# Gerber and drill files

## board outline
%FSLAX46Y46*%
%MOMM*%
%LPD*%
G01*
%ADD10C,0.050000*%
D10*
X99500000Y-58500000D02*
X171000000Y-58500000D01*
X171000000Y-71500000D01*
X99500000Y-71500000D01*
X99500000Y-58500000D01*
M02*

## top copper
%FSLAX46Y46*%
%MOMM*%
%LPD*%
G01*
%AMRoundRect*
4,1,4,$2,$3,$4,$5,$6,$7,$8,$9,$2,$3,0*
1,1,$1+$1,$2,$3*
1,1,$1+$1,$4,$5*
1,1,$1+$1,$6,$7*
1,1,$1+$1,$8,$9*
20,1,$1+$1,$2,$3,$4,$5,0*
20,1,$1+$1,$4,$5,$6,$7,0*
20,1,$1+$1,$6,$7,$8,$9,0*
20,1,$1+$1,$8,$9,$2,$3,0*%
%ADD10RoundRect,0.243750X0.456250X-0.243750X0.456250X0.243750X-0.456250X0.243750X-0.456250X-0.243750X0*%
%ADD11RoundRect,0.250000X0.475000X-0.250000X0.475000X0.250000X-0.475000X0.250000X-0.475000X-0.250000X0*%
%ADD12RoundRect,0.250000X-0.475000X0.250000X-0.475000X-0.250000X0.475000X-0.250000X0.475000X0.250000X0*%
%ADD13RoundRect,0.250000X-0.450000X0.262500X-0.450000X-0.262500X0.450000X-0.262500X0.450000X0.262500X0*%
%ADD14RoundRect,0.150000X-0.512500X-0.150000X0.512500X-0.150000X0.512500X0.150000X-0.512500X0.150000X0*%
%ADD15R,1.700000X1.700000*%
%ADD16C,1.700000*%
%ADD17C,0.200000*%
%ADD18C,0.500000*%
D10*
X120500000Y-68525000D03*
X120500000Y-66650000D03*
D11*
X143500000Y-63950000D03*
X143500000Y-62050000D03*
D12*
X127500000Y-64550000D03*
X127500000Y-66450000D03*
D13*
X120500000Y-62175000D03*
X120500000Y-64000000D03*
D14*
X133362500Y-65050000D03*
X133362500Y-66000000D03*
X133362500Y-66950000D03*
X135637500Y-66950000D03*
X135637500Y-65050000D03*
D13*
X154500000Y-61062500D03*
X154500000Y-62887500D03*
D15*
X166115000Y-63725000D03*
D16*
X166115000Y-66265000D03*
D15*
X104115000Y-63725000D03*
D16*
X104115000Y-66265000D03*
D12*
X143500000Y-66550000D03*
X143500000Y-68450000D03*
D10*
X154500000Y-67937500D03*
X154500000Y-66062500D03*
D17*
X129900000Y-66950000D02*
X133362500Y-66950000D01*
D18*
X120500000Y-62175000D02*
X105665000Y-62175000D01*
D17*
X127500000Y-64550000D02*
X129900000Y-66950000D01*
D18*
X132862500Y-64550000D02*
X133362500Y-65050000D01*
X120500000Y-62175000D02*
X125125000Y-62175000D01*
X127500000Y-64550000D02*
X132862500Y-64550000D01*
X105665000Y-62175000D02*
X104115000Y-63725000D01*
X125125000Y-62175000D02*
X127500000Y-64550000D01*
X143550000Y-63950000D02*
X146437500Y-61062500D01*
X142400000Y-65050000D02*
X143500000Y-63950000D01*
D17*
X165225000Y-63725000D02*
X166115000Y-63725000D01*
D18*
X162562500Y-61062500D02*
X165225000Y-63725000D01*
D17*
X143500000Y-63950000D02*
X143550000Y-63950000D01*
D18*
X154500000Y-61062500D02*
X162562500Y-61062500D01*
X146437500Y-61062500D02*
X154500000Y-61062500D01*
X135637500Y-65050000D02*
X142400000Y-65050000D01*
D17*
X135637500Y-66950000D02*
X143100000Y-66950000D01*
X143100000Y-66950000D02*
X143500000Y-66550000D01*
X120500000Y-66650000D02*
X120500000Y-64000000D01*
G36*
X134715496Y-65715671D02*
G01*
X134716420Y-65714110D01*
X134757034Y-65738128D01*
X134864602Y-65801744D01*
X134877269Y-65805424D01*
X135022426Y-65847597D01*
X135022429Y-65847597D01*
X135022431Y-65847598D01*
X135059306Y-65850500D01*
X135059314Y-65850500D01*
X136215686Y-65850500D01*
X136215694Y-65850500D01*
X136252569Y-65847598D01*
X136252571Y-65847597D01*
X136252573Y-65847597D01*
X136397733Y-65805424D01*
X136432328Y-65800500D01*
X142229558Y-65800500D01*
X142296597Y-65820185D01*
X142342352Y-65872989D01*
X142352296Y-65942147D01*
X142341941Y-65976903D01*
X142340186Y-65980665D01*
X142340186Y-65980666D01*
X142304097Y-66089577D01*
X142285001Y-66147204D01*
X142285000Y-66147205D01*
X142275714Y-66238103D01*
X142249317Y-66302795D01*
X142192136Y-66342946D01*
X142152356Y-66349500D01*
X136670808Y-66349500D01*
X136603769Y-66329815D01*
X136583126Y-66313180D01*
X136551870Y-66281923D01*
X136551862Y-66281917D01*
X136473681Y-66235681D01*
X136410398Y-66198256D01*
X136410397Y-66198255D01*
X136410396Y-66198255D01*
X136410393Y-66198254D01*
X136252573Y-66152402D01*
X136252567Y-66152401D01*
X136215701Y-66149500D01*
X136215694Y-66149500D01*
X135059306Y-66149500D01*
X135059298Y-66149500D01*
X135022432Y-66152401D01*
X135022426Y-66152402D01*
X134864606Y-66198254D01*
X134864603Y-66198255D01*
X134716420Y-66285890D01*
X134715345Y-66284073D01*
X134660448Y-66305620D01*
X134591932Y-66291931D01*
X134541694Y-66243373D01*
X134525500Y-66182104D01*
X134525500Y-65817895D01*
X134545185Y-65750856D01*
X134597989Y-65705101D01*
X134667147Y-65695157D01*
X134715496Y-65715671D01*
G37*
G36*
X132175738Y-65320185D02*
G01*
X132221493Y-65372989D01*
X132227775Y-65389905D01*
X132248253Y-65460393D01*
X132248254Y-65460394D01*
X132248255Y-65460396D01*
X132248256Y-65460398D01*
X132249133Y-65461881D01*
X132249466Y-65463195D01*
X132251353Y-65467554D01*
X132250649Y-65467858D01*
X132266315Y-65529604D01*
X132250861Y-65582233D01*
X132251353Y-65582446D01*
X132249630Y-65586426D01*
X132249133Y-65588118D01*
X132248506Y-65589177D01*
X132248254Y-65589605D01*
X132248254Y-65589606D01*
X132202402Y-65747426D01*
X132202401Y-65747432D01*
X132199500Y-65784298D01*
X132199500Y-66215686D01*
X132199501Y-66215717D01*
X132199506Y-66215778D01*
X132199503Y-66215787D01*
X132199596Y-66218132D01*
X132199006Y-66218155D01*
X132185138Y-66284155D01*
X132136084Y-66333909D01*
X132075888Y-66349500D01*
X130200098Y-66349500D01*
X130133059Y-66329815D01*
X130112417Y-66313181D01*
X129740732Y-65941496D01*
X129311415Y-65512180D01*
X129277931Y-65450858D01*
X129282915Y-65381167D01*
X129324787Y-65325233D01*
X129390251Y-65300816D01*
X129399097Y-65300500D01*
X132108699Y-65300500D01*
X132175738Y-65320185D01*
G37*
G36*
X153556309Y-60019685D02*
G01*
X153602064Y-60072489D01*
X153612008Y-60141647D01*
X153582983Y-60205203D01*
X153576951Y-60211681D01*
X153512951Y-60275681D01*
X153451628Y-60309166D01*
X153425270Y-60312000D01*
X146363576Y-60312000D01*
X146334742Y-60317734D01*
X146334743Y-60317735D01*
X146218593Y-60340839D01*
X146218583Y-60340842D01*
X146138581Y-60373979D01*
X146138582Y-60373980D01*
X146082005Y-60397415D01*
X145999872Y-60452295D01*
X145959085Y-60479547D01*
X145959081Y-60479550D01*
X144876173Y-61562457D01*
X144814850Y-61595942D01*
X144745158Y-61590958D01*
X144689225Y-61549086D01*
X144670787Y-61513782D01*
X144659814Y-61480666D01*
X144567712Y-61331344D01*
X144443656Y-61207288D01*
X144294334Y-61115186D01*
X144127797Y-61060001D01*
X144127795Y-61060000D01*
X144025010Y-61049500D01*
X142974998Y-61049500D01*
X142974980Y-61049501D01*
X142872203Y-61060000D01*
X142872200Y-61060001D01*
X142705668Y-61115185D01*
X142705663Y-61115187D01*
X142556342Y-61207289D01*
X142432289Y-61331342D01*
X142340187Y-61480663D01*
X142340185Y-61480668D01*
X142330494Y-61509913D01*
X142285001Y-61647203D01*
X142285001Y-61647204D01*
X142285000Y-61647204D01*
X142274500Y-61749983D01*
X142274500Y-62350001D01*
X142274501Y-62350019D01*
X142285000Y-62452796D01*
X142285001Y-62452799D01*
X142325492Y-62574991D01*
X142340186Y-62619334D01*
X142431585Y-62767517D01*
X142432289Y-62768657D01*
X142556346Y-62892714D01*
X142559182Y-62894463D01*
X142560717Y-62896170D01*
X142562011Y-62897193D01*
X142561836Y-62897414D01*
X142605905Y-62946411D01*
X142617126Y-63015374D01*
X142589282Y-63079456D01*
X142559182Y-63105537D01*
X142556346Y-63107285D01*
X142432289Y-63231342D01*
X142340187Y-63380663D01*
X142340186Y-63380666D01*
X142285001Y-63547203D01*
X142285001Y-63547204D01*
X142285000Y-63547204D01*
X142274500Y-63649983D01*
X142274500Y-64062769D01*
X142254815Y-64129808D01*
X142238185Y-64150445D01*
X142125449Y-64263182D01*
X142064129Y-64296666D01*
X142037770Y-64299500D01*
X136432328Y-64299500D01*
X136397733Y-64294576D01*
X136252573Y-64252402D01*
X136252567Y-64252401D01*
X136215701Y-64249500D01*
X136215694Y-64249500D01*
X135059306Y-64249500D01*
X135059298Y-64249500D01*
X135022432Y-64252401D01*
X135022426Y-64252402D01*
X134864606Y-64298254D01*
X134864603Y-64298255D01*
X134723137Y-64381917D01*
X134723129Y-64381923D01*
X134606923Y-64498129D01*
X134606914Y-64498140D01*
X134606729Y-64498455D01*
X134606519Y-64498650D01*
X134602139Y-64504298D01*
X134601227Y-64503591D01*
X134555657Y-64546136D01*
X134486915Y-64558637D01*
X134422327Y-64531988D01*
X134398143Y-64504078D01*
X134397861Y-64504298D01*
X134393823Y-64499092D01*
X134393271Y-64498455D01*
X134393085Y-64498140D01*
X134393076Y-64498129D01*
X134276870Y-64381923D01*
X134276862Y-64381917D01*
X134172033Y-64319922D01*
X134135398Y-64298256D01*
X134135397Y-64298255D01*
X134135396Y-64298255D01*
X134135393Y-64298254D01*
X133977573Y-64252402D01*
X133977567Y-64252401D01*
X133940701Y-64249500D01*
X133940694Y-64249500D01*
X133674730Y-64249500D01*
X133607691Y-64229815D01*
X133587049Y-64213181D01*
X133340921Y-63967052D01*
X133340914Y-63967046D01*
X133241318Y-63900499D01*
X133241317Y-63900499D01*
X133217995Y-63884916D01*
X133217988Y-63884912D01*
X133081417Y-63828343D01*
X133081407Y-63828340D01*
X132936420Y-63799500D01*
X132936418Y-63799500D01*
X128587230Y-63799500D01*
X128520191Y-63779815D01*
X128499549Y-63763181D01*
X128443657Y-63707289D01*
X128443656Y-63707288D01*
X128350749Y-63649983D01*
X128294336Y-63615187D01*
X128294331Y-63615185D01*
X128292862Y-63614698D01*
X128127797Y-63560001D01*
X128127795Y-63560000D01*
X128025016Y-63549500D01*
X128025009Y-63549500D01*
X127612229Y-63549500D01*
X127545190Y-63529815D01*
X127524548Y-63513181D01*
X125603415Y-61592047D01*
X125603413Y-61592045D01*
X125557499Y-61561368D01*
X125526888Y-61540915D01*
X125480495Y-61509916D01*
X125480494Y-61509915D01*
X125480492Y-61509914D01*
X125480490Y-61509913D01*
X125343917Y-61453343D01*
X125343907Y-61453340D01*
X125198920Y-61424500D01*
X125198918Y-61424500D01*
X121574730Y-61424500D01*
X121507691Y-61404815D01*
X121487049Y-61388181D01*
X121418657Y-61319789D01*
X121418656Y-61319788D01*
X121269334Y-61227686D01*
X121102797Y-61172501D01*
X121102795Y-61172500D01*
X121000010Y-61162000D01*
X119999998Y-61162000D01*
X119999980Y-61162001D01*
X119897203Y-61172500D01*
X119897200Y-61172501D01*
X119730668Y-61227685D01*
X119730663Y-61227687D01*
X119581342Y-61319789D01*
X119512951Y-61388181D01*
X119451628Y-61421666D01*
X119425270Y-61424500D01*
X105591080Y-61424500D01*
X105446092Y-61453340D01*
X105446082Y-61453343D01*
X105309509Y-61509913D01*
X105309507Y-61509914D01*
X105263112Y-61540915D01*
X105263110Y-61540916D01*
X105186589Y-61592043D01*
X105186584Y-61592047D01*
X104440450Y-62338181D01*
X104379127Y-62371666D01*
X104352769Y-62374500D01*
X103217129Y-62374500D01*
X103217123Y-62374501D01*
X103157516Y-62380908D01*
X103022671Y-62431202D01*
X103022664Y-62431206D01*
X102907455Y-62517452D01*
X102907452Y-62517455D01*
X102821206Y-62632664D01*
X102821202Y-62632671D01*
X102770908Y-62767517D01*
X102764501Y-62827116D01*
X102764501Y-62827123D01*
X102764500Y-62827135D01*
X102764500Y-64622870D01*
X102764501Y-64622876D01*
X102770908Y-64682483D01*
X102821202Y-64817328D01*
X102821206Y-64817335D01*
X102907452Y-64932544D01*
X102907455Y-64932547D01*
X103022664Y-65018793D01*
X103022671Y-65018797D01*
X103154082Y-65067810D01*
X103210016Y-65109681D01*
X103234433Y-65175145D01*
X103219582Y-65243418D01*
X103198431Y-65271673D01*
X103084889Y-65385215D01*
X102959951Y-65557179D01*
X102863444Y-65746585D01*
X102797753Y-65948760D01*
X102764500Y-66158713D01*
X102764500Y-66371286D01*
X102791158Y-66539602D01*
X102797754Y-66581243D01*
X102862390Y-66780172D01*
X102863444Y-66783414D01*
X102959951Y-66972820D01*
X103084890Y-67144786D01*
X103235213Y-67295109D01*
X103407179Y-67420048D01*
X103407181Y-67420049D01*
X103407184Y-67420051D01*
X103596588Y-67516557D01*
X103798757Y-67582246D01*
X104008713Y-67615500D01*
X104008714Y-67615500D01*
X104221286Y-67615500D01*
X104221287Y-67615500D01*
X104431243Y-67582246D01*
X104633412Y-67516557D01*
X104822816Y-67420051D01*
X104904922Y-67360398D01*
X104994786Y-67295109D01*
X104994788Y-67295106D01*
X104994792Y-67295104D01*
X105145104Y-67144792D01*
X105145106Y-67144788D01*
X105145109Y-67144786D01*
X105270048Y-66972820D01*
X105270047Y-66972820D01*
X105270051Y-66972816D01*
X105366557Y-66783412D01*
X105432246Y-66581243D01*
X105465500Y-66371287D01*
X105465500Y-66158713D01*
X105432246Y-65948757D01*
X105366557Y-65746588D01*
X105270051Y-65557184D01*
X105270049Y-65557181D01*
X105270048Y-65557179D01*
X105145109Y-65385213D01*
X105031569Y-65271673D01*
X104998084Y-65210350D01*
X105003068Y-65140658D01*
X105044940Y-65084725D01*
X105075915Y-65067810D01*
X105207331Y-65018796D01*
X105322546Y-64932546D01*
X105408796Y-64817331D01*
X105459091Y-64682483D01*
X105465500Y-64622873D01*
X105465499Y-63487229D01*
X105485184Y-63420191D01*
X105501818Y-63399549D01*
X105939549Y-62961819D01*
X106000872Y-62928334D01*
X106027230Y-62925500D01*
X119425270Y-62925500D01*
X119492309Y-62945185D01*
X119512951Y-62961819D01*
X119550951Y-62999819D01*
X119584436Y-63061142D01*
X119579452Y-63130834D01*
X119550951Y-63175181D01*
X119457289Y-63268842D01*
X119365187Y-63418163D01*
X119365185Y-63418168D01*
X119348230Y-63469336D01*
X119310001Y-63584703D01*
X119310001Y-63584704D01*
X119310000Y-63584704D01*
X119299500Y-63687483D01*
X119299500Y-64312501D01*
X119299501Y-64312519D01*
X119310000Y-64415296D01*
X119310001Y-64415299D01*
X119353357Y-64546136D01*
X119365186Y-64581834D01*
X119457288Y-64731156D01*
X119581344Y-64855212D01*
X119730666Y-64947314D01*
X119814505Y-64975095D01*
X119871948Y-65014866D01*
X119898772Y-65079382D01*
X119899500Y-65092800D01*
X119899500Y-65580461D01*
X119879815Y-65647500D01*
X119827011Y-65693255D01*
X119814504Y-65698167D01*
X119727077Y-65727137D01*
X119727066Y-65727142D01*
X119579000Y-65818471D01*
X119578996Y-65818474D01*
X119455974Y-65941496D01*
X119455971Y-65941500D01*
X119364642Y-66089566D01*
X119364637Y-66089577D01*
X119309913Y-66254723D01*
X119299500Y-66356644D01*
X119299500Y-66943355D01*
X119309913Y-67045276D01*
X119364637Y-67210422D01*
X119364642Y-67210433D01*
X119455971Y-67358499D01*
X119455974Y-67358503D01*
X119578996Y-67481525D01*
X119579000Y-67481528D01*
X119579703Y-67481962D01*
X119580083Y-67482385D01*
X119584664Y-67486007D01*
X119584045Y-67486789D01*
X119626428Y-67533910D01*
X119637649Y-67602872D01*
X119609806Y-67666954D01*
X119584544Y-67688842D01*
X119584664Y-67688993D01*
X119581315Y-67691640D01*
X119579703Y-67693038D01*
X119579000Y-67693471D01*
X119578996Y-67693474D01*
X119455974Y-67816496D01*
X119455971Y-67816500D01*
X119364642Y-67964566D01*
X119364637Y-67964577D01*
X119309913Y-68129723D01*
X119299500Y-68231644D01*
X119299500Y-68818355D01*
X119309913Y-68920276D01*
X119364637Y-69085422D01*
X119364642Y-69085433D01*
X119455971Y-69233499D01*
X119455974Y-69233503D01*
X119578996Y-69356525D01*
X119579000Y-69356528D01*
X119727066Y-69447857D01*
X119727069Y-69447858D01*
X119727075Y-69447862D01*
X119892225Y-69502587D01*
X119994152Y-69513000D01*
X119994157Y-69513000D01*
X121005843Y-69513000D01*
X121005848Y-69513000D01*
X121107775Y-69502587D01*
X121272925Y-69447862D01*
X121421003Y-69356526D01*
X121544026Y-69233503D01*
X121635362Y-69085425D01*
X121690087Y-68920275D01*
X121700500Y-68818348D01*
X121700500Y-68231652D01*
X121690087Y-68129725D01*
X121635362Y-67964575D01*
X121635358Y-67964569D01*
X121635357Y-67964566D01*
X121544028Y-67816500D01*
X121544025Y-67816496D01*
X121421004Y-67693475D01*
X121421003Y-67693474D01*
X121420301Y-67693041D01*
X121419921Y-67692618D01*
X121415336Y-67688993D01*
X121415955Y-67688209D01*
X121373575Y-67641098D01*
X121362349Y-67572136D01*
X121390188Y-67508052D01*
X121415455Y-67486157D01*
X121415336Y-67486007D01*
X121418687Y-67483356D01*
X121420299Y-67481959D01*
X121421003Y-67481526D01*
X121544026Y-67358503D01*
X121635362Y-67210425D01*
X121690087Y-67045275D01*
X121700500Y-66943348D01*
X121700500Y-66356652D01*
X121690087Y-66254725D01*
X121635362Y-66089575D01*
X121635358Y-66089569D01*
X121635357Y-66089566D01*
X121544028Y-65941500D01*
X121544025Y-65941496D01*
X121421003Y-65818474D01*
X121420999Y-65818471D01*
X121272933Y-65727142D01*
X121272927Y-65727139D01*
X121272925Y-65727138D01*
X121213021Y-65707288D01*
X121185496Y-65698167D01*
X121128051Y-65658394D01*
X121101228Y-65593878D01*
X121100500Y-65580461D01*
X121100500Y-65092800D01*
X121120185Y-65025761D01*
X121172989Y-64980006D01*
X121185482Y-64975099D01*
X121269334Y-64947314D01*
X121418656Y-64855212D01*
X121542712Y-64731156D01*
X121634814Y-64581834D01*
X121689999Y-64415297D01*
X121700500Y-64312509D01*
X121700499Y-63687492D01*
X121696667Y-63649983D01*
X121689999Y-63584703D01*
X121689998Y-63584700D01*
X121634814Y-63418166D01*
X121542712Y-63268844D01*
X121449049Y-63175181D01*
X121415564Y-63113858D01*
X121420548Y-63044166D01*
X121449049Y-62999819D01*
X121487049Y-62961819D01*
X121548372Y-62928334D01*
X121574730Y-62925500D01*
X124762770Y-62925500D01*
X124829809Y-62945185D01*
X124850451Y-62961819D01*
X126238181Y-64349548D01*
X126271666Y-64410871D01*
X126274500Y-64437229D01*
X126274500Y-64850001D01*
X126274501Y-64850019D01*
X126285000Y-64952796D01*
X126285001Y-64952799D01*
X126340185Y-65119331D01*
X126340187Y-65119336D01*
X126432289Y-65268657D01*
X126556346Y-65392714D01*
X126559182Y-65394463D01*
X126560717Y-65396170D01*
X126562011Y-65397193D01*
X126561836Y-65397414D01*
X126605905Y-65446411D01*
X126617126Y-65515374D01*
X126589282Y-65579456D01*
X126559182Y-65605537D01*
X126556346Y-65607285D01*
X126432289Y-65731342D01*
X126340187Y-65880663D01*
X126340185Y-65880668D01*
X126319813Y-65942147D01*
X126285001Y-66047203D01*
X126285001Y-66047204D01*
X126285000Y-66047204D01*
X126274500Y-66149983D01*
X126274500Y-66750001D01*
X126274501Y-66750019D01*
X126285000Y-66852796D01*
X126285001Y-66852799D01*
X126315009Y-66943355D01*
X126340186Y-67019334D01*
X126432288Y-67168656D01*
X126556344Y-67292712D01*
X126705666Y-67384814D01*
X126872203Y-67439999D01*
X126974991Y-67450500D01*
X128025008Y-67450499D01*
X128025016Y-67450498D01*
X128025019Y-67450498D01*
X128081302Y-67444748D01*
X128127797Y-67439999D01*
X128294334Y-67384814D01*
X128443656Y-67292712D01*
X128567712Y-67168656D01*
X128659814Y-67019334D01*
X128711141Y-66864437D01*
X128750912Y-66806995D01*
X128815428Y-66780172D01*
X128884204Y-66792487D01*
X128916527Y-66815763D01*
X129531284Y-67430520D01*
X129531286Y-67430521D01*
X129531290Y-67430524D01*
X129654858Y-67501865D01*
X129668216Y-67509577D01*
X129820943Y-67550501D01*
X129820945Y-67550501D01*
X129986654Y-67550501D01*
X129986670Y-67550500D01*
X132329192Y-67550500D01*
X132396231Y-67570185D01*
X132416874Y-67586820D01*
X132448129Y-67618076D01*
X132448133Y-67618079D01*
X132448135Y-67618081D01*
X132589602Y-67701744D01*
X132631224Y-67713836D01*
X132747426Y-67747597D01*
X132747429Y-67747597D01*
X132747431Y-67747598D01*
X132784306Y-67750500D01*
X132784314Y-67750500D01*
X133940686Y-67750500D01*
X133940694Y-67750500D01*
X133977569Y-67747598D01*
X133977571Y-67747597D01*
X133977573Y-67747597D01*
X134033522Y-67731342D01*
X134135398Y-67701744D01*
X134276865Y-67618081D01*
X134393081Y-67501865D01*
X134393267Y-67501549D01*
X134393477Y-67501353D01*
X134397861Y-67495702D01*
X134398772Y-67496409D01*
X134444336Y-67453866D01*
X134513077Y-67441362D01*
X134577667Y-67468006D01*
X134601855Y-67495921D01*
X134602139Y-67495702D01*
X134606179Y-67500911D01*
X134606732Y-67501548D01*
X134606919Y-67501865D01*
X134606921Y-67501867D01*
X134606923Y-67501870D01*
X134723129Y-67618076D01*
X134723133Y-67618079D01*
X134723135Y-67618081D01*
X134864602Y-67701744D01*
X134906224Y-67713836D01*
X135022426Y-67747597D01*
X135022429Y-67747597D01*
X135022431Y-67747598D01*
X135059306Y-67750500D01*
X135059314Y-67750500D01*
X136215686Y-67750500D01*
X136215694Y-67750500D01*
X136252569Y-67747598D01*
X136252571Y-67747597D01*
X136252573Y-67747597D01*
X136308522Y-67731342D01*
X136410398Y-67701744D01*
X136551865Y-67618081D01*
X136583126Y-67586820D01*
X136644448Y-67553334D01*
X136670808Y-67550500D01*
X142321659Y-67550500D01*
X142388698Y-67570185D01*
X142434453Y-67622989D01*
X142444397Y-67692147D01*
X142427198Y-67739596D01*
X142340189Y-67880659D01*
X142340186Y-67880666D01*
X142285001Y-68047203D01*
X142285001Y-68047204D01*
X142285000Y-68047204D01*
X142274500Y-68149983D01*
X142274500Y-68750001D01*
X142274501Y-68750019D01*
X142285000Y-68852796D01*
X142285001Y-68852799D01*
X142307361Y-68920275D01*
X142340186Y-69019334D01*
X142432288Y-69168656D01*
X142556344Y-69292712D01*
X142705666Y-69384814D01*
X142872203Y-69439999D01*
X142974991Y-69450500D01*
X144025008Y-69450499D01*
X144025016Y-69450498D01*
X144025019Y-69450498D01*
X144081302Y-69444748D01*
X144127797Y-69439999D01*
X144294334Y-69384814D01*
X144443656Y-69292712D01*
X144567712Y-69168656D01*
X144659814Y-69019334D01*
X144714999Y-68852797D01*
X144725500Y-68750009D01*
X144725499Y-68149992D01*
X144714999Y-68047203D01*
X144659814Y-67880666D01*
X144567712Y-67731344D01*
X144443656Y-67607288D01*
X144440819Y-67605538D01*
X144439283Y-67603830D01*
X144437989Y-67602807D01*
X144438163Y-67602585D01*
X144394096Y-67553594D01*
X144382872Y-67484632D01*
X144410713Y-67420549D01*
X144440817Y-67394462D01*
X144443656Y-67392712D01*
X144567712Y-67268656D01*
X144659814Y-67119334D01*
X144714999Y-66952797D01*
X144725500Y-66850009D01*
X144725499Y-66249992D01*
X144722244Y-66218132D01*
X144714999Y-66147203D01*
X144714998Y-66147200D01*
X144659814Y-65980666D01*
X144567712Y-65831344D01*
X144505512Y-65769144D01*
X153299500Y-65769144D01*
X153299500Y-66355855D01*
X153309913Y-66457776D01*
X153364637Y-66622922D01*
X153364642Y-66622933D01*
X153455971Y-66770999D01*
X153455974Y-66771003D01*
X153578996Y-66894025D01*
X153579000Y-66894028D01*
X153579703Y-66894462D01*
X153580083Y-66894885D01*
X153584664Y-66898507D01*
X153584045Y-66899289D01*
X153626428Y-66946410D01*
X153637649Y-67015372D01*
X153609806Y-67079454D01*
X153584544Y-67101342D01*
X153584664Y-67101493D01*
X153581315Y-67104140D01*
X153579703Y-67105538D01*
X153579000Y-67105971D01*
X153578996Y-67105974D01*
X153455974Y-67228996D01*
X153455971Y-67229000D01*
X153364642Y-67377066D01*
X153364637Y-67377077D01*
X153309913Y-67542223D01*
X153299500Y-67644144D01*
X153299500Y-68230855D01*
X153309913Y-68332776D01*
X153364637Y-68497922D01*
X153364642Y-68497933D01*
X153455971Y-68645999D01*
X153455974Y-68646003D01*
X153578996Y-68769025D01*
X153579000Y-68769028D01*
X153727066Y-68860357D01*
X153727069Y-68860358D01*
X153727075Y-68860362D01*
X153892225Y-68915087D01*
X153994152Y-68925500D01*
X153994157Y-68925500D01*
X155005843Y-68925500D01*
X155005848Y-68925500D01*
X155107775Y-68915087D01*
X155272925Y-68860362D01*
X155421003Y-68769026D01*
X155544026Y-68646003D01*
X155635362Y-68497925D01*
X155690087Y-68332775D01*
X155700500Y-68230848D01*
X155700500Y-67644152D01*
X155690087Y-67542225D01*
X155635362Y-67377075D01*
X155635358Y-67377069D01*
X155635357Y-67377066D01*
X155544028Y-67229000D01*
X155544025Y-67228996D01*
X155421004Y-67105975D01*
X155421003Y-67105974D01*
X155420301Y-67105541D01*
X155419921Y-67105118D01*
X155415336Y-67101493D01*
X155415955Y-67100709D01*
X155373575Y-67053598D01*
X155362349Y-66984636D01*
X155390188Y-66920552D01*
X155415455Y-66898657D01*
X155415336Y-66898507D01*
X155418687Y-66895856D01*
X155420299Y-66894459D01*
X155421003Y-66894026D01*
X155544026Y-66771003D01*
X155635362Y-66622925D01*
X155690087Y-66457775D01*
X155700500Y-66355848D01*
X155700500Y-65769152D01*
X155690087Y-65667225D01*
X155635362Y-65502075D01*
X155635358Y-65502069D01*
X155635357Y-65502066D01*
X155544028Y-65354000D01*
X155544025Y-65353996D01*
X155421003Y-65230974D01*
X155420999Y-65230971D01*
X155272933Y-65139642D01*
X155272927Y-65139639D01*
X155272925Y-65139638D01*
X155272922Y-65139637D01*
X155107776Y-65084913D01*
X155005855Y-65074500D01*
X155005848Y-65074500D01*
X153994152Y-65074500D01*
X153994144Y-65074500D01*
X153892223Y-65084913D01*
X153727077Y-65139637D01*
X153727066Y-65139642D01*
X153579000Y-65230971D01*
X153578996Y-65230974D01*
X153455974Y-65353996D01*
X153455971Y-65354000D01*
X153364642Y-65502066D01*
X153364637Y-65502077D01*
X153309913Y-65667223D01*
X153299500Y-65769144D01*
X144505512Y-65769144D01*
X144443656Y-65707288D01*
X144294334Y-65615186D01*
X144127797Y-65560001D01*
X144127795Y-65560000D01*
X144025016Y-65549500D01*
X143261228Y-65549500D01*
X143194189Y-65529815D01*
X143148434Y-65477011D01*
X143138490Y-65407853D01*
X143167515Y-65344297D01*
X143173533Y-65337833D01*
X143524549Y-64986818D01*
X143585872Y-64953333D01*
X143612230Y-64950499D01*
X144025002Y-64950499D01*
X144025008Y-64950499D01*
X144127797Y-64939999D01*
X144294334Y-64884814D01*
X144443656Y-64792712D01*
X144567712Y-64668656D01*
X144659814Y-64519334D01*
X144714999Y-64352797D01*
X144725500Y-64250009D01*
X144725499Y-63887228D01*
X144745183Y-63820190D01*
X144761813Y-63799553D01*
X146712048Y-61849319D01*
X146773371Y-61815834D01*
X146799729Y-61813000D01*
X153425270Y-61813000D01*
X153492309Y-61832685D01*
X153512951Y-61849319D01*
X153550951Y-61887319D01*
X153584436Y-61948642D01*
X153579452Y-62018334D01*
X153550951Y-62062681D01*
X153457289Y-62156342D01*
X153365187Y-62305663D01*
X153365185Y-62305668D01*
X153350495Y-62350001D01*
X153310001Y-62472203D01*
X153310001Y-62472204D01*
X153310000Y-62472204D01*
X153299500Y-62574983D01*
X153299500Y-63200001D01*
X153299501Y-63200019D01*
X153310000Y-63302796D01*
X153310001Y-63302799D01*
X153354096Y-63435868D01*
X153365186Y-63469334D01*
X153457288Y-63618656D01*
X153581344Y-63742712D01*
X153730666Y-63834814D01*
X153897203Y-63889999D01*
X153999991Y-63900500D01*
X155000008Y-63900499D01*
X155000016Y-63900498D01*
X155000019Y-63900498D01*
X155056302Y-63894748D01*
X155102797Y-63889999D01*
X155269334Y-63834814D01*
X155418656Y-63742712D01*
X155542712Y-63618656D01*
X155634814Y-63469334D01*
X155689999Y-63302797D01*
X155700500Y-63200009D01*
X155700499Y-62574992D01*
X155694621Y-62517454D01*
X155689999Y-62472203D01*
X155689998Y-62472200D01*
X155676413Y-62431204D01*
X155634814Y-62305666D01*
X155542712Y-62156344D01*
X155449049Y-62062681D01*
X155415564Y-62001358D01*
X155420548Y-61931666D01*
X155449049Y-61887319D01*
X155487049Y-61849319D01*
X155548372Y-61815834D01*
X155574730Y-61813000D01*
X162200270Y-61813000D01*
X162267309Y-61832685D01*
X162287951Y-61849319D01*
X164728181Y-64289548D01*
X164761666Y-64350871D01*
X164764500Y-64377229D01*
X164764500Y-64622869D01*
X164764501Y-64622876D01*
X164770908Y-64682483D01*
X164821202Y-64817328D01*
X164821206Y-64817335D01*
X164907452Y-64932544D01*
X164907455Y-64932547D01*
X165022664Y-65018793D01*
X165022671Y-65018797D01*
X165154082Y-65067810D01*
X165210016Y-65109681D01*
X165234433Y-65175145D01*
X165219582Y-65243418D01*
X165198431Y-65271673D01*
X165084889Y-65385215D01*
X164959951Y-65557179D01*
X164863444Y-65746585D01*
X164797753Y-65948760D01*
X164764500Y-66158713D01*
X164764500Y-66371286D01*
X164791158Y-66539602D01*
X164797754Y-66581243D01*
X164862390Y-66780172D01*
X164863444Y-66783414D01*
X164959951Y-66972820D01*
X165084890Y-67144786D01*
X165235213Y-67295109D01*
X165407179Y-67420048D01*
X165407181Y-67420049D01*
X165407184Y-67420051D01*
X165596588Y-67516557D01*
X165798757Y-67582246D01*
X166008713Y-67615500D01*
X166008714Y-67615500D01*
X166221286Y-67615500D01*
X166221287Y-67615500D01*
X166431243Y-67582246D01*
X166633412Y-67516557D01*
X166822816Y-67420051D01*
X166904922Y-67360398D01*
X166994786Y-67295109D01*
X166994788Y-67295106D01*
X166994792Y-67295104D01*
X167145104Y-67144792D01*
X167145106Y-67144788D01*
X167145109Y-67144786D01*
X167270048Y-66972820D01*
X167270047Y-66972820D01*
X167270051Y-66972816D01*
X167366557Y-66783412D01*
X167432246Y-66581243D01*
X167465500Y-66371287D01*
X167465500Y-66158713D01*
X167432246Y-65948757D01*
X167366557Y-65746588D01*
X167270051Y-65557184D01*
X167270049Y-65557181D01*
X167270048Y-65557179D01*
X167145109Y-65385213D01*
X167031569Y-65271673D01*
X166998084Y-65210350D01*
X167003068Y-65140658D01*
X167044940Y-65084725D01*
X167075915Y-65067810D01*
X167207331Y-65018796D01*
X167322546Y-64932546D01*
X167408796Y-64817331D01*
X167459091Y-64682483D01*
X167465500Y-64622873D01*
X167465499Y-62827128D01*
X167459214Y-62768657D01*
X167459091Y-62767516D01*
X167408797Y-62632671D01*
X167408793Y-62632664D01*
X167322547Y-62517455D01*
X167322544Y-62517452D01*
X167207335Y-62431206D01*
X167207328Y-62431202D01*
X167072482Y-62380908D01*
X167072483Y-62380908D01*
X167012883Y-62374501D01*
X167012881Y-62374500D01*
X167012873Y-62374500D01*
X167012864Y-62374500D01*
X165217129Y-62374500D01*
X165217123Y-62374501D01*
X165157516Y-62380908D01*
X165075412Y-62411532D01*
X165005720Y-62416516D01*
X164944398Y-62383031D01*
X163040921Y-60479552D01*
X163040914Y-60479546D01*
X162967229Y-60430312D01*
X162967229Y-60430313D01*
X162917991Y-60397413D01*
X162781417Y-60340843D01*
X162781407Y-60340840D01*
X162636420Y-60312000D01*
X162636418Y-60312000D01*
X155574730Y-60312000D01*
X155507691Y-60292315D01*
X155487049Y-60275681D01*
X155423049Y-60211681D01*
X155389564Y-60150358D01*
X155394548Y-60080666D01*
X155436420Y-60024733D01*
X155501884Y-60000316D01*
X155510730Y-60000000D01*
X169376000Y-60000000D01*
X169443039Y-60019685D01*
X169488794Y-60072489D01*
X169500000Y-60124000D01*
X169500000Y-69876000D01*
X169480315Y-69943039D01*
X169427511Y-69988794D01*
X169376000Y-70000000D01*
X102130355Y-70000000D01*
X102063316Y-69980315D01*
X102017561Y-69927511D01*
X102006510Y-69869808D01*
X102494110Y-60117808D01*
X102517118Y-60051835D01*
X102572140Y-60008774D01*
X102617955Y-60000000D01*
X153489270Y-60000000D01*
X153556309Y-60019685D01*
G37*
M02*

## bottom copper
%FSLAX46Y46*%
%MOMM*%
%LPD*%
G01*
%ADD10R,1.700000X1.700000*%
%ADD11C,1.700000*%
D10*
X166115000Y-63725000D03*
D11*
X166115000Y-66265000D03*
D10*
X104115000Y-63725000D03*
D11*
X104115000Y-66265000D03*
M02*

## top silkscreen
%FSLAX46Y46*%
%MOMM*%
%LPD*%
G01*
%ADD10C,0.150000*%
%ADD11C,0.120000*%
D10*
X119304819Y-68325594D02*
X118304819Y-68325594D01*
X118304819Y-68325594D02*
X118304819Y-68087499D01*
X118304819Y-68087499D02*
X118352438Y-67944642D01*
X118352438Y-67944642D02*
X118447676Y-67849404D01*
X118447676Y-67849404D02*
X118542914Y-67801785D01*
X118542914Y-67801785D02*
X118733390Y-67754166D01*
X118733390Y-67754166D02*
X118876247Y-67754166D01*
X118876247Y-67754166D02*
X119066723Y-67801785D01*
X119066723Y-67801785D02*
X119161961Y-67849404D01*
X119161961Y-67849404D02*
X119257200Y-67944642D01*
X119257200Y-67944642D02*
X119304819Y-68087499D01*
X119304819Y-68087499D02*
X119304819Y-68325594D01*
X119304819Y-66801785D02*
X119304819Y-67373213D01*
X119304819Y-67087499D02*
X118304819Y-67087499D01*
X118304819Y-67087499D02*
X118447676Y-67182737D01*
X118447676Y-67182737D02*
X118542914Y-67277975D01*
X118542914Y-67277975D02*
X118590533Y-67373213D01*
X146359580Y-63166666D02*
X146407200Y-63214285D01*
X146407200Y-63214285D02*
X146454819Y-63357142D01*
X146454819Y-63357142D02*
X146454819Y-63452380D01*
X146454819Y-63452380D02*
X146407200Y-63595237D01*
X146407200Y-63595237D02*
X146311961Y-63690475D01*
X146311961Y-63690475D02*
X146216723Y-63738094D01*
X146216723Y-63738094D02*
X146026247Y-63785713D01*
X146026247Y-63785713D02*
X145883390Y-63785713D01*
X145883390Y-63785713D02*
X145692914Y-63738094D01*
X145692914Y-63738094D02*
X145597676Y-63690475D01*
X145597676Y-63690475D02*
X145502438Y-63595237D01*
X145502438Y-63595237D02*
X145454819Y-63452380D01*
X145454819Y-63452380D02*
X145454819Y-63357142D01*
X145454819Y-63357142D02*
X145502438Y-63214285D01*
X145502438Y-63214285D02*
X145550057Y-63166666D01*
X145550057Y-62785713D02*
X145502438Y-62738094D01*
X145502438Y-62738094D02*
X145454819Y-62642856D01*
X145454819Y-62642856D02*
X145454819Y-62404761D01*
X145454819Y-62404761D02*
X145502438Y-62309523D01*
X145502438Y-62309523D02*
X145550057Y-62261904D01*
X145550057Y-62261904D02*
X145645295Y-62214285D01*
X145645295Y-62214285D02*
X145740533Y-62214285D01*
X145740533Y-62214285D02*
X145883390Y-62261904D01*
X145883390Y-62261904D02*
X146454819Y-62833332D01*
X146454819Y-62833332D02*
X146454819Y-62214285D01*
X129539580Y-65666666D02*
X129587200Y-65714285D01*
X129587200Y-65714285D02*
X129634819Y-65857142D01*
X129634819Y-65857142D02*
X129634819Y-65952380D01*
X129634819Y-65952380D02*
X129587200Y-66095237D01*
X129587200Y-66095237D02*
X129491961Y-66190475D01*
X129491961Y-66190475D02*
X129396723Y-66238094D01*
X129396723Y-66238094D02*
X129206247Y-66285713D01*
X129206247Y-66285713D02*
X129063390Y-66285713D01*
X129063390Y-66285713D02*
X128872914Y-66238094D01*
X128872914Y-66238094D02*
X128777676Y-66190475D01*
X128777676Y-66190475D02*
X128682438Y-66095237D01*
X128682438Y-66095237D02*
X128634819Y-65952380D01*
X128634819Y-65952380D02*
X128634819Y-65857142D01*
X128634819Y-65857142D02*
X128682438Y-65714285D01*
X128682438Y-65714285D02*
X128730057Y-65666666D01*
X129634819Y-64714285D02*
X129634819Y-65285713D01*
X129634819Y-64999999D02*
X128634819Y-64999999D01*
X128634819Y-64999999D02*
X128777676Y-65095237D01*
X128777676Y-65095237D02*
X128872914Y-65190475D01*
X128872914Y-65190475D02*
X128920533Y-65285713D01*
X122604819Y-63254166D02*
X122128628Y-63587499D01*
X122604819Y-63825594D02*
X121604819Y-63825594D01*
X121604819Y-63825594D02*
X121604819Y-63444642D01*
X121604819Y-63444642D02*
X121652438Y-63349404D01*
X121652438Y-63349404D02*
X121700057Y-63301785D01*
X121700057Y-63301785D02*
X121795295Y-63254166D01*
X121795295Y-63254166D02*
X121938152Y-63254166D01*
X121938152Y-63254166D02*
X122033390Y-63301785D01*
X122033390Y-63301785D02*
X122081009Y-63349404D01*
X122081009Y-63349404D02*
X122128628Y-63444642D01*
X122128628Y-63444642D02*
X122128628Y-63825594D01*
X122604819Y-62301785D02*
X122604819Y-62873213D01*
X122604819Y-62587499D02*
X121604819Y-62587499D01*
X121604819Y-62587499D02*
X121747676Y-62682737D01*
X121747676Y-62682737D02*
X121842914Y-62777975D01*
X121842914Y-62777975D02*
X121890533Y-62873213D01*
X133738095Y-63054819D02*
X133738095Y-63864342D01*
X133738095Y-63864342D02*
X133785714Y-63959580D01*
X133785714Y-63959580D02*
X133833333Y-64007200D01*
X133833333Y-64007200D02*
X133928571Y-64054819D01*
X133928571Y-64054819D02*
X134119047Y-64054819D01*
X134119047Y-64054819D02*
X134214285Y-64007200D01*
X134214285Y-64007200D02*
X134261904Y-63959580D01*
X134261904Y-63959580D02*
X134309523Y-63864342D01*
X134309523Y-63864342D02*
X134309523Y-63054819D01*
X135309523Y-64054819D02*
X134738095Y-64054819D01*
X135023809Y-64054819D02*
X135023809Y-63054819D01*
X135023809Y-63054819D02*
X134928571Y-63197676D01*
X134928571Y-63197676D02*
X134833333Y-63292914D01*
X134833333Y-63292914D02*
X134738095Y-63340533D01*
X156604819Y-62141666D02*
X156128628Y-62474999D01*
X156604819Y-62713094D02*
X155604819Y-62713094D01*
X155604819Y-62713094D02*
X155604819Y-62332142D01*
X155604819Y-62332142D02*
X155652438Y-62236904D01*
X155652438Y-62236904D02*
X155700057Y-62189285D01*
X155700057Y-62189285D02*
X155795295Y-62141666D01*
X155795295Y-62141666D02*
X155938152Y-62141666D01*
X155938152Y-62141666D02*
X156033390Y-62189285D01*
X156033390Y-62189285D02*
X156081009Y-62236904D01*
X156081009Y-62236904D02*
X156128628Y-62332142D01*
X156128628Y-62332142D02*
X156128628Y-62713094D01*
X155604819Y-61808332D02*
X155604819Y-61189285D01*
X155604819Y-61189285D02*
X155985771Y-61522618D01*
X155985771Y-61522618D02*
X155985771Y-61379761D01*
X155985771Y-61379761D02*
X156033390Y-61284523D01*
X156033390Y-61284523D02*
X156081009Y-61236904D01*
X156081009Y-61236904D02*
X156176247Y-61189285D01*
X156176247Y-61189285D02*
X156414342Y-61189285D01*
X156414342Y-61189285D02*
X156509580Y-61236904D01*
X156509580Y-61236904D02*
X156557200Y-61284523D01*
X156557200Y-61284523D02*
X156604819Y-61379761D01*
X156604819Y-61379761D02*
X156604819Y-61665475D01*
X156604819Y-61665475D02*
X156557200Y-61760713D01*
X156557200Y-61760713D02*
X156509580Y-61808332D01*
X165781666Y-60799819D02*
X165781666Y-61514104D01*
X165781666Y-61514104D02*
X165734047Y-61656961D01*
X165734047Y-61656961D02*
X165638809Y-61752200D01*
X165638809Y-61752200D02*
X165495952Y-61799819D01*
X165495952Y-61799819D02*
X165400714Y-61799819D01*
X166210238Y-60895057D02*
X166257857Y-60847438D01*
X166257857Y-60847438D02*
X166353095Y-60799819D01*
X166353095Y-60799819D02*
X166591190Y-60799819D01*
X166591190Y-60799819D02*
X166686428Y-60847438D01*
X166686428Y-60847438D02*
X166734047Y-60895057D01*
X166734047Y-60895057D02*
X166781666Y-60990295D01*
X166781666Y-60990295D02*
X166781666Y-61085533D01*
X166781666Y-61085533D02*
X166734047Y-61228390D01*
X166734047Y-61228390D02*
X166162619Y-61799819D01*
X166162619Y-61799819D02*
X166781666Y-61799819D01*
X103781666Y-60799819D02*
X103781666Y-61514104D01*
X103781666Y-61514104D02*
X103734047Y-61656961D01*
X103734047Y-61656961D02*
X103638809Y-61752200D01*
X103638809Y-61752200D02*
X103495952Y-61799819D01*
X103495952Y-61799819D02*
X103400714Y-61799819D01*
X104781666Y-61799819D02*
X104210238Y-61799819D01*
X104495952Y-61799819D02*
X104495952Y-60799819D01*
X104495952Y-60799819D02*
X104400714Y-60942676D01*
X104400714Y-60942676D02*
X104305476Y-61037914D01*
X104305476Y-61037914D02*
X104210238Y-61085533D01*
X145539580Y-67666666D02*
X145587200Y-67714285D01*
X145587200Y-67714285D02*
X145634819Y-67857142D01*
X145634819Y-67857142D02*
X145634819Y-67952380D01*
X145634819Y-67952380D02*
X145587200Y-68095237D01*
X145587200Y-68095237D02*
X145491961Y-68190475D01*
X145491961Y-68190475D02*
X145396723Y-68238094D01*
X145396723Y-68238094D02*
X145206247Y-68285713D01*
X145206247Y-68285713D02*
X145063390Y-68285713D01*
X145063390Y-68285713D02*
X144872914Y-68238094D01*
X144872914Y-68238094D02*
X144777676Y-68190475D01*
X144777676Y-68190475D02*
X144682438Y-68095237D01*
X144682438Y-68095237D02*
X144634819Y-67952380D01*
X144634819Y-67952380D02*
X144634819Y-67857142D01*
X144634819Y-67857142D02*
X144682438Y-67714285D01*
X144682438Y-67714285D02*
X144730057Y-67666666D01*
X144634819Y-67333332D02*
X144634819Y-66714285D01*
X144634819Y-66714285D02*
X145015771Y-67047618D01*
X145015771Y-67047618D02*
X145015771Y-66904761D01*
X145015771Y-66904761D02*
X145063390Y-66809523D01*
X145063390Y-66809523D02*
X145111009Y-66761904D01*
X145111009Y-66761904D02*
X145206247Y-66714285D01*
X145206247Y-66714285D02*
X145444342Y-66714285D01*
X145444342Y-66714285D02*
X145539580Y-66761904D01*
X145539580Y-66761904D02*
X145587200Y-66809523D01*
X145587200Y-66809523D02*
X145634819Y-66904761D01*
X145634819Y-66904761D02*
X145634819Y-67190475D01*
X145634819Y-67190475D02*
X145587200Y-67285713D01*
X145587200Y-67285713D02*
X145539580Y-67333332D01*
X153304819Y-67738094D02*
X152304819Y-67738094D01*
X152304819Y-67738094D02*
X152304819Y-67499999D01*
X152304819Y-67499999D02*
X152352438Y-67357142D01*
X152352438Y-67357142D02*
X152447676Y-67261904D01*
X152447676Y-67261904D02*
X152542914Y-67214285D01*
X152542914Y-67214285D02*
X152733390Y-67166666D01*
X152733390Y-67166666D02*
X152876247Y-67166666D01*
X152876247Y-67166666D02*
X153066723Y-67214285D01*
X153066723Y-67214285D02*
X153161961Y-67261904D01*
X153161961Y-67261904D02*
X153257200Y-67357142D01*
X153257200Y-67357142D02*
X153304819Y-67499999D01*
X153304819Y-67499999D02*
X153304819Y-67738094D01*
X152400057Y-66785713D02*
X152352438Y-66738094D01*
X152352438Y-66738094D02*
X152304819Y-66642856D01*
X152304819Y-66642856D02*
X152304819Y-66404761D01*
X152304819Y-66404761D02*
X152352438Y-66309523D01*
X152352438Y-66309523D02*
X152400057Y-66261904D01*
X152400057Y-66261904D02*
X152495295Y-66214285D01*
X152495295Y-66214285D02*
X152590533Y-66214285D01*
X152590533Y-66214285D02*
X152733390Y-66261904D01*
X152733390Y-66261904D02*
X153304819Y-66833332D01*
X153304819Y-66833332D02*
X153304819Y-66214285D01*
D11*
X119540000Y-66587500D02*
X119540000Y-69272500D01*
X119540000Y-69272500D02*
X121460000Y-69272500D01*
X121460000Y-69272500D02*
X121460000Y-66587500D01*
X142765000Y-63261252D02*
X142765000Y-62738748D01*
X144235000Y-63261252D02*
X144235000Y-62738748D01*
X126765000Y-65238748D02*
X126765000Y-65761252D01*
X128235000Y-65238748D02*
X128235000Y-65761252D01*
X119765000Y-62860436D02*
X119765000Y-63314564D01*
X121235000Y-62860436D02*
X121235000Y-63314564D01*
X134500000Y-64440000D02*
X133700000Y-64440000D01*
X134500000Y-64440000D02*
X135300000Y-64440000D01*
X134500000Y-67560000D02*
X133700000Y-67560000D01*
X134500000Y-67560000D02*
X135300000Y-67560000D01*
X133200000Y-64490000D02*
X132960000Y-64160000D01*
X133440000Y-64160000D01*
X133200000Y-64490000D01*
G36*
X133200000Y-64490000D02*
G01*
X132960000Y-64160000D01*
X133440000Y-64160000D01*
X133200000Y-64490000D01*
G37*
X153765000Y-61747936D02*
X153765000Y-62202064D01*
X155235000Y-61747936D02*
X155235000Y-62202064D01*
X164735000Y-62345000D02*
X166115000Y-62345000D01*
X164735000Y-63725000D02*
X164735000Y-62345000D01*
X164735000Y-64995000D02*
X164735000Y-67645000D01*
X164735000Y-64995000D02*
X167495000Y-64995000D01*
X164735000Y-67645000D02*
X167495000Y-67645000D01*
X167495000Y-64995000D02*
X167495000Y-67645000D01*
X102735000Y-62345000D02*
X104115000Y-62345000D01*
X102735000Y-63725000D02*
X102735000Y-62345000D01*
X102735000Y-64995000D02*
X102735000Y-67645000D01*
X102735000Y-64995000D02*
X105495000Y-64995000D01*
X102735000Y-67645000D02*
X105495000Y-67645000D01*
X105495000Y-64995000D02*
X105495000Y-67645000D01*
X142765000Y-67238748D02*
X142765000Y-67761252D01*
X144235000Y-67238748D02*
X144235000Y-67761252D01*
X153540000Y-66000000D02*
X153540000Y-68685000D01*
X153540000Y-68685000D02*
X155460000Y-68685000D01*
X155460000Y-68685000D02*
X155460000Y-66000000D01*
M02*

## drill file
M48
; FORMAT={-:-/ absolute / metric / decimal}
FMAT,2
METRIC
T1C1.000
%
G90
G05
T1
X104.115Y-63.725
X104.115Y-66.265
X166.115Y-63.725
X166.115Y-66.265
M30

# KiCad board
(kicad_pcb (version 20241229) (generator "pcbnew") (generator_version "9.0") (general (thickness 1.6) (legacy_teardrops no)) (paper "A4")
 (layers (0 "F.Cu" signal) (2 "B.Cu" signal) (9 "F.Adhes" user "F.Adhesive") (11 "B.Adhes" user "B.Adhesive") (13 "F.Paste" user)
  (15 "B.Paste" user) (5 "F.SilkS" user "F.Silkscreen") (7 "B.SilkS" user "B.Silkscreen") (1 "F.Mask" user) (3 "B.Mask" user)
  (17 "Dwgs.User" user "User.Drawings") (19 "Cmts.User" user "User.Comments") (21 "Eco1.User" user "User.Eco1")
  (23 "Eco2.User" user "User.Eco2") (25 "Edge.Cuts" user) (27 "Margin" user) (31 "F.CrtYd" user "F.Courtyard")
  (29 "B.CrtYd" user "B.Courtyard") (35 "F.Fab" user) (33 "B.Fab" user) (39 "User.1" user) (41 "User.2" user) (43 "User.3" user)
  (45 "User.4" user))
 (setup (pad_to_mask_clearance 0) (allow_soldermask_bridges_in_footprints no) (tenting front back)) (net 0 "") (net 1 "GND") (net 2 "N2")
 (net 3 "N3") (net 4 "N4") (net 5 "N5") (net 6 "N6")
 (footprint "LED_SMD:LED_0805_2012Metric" (layer "F.Cu") (at 120.5 67.5875 90)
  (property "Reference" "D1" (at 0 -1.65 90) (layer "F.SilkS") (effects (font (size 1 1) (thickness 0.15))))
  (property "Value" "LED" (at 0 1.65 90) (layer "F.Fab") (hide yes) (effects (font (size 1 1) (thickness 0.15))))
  (fp_line (start 1 -0.96) (end -1.685 -0.96) (stroke (width 0.12) (type solid)) (layer "F.SilkS"))
  (fp_line (start -1.685 -0.96) (end -1.685 0.96) (stroke (width 0.12) (type solid)) (layer "F.SilkS"))
  (fp_line (start -1.685 0.96) (end 1 0.96) (stroke (width 0.12) (type solid)) (layer "F.SilkS"))
  (pad "1" smd roundrect (at -0.9375 0 90) (size 0.975 1.4) (layers "F.Cu" "F.Mask" "F.Paste") (roundrect_rratio 0.25) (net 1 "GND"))
  (pad "2" smd roundrect (at 0.9375 0 90) (size 0.975 1.4) (layers "F.Cu" "F.Mask" "F.Paste") (roundrect_rratio 0.25) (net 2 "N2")))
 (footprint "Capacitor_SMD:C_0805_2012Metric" (layer "F.Cu") (at 143.5 63 90)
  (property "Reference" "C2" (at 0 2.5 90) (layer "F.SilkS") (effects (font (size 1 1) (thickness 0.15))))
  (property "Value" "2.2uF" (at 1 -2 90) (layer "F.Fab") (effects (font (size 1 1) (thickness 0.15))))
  (fp_line (start -0.261252 -0.735) (end 0.261252 -0.735) (stroke (width 0.12) (type solid)) (layer "F.SilkS"))
  (fp_line (start -0.261252 0.735) (end 0.261252 0.735) (stroke (width 0.12) (type solid)) (layer "F.SilkS"))
  (pad "1" smd roundrect (at -0.95 0 90) (size 1 1.45) (layers "F.Cu" "F.Mask" "F.Paste") (roundrect_rratio 0.25) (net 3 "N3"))
  (pad "2" smd roundrect (at 0.95 0 90) (size 1 1.45) (layers "F.Cu" "F.Mask" "F.Paste") (roundrect_rratio 0.25) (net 1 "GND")))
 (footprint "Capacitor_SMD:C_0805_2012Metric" (layer "F.Cu") (at 127.5 65.5 -90)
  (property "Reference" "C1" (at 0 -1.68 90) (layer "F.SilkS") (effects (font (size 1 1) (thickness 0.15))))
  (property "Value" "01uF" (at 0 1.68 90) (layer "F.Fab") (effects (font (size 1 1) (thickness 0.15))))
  (fp_line (start -0.261252 0.735) (end 0.261252 0.735) (stroke (width 0.12) (type solid)) (layer "F.SilkS"))
  (fp_line (start -0.261252 -0.735) (end 0.261252 -0.735) (stroke (width 0.12) (type solid)) (layer "F.SilkS"))
  (pad "1" smd roundrect (at -0.95 0 270) (size 1 1.45) (layers "F.Cu" "F.Mask" "F.Paste") (roundrect_rratio 0.25) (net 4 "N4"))
  (pad "2" smd roundrect (at 0.95 0 270) (size 1 1.45) (layers "F.Cu" "F.Mask" "F.Paste") (roundrect_rratio 0.25) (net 1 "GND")))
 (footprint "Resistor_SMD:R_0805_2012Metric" (layer "F.Cu") (at 120.5 63.0875 -90)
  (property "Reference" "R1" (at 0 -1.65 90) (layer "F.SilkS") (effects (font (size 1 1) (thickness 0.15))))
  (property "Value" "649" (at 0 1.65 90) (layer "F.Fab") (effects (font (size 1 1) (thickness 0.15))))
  (fp_line (start -0.227064 0.735) (end 0.227064 0.735) (stroke (width 0.12) (type solid)) (layer "F.SilkS"))
  (fp_line (start -0.227064 -0.735) (end 0.227064 -0.735) (stroke (width 0.12) (type solid)) (layer "F.SilkS"))
  (pad "1" smd roundrect (at -0.9125 0 270) (size 1.025 1.4) (layers "F.Cu" "F.Mask" "F.Paste") (roundrect_rratio 0.243902) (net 4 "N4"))
  (pad "2" smd roundrect (at 0.9125 0 270) (size 1.025 1.4) (layers "F.Cu" "F.Mask" "F.Paste") (roundrect_rratio 0.243902) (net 2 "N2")))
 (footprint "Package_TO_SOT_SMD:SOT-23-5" (layer "F.Cu") (at 134.5 66)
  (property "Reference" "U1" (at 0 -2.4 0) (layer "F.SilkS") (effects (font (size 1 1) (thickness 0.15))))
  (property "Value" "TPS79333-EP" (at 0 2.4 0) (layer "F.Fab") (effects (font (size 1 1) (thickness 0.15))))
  (fp_line (start 0 -1.56) (end -0.8 -1.56) (stroke (width 0.12) (type solid)) (layer "F.SilkS"))
  (fp_line (start 0 -1.56) (end 0.8 -1.56) (stroke (width 0.12) (type solid)) (layer "F.SilkS"))
  (fp_line (start 0 1.56) (end -0.8 1.56) (stroke (width 0.12) (type solid)) (layer "F.SilkS"))
  (fp_line (start 0 1.56) (end 0.8 1.56) (stroke (width 0.12) (type solid)) (layer "F.SilkS"))
  (fp_poly (pts (xy -1.3 -1.51) (xy -1.54 -1.84) (xy -1.06 -1.84)) (stroke (width 0.12) (type solid)) (fill yes) (layer "F.SilkS"))
  (pad "1" smd roundrect (at -1.1375 -0.95) (size 1.325 0.6) (layers "F.Cu" "F.Mask" "F.Paste") (roundrect_rratio 0.25) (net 4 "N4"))
  (pad "2" smd roundrect (at -1.1375 0) (size 1.325 0.6) (layers "F.Cu" "F.Mask" "F.Paste") (roundrect_rratio 0.25) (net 1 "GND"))
  (pad "3" smd roundrect (at -1.1375 0.95) (size 1.325 0.6) (layers "F.Cu" "F.Mask" "F.Paste") (roundrect_rratio 0.25) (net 4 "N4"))
  (pad "4" smd roundrect (at 1.1375 0.95) (size 1.325 0.6) (layers "F.Cu" "F.Mask" "F.Paste") (roundrect_rratio 0.25) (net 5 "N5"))
  (pad "5" smd roundrect (at 1.1375 -0.95) (size 1.325 0.6) (layers "F.Cu" "F.Mask" "F.Paste") (roundrect_rratio 0.25) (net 3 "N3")))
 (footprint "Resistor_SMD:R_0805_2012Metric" (layer "F.Cu") (at 154.5 61.975 -90)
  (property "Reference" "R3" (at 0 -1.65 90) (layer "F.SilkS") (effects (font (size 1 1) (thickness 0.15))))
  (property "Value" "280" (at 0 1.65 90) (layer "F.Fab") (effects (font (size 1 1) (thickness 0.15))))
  (fp_line (start -0.227064 0.735) (end 0.227064 0.735) (stroke (width 0.12) (type solid)) (layer "F.SilkS"))
  (fp_line (start -0.227064 -0.735) (end 0.227064 -0.735) (stroke (width 0.12) (type solid)) (layer "F.SilkS"))
  (pad "1" smd roundrect (at -0.9125 0 270) (size 1.025 1.4) (layers "F.Cu" "F.Mask" "F.Paste") (roundrect_rratio 0.243902) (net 3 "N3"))
  (pad "2" smd roundrect (at 0.9125 0 270) (size 1.025 1.4) (layers "F.Cu" "F.Mask" "F.Paste") (roundrect_rratio 0.243902) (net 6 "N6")))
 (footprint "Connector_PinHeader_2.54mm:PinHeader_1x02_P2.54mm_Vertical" (layer "F.Cu") (at 166.115 63.725)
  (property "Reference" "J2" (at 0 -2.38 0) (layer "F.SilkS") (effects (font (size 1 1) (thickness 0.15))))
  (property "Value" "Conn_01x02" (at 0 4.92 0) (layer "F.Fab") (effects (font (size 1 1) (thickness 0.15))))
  (fp_line (start -1.38 -1.38) (end 0 -1.38) (stroke (width 0.12) (type solid)) (layer "F.SilkS"))
  (fp_line (start -1.38 0) (end -1.38 -1.38) (stroke (width 0.12) (type solid)) (layer "F.SilkS"))
  (fp_line (start -1.38 1.27) (end -1.38 3.92) (stroke (width 0.12) (type solid)) (layer "F.SilkS"))
  (fp_line (start -1.38 1.27) (end 1.38 1.27) (stroke (width 0.12) (type solid)) (layer "F.SilkS"))
  (fp_line (start -1.38 3.92) (end 1.38 3.92) (stroke (width 0.12) (type solid)) (layer "F.SilkS"))
  (fp_line (start 1.38 1.27) (end 1.38 3.92) (stroke (width 0.12) (type solid)) (layer "F.SilkS"))
  (pad "1" thru_hole rect (at 0 0) (size 1.7 1.7) (drill 1) (layers "*.Cu" "*.Mask") (remove_unused_layers no) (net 3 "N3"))
  (pad "2" thru_hole circle (at 0 2.54) (size 1.7 1.7) (drill 1) (layers "*.Cu" "*.Mask") (remove_unused_layers no) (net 1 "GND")))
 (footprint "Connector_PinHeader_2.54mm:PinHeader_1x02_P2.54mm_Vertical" (layer "F.Cu") (at 104.115 63.725)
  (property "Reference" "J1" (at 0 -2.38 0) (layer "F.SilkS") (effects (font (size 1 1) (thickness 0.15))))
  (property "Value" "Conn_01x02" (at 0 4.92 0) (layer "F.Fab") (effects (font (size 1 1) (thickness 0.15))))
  (fp_line (start -1.38 -1.38) (end 0 -1.38) (stroke (width 0.12) (type solid)) (layer "F.SilkS"))
  (fp_line (start -1.38 0) (end -1.38 -1.38) (stroke (width 0.12) (type solid)) (layer "F.SilkS"))
  (fp_line (start -1.38 1.27) (end -1.38 3.92) (stroke (width 0.12) (type solid)) (layer "F.SilkS"))
  (fp_line (start -1.38 1.27) (end 1.38 1.27) (stroke (width 0.12) (type solid)) (layer "F.SilkS"))
  (fp_line (start -1.38 3.92) (end 1.38 3.92) (stroke (width 0.12) (type solid)) (layer "F.SilkS"))
  (fp_line (start 1.38 1.27) (end 1.38 3.92) (stroke (width 0.12) (type solid)) (layer "F.SilkS"))
  (pad "1" thru_hole rect (at 0 0) (size 1.7 1.7) (drill 1) (layers "*.Cu" "*.Mask") (remove_unused_layers no) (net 4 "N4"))
  (pad "2" thru_hole circle (at 0 2.54) (size 1.7 1.7) (drill 1) (layers "*.Cu" "*.Mask") (remove_unused_layers no) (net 1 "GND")))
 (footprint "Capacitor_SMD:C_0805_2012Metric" (layer "F.Cu") (at 143.5 67.5 -90)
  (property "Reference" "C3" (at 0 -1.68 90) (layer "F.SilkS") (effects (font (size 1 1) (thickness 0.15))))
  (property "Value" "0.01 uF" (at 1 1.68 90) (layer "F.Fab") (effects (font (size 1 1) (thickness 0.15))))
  (fp_line (start -0.261252 0.735) (end 0.261252 0.735) (stroke (width 0.12) (type solid)) (layer "F.SilkS"))
  (fp_line (start -0.261252 -0.735) (end 0.261252 -0.735) (stroke (width 0.12) (type solid)) (layer "F.SilkS"))
  (pad "1" smd roundrect (at -0.95 0 270) (size 1 1.45) (layers "F.Cu" "F.Mask" "F.Paste") (roundrect_rratio 0.25) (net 5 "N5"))
  (pad "2" smd roundrect (at 0.95 0 270) (size 1 1.45) (layers "F.Cu" "F.Mask" "F.Paste") (roundrect_rratio 0.25) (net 1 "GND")))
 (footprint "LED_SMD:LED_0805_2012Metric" (layer "F.Cu") (at 154.5 67 90)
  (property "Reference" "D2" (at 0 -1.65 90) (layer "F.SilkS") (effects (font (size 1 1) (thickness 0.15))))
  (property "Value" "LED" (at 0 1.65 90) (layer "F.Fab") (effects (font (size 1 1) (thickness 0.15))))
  (fp_line (start 1 -0.96) (end -1.685 -0.96) (stroke (width 0.12) (type solid)) (layer "F.SilkS"))
  (fp_line (start -1.685 -0.96) (end -1.685 0.96) (stroke (width 0.12) (type solid)) (layer "F.SilkS"))
  (fp_line (start -1.685 0.96) (end 1 0.96) (stroke (width 0.12) (type solid)) (layer "F.SilkS"))
  (pad "1" smd roundrect (at -0.9375 0 90) (size 0.975 1.4) (layers "F.Cu" "F.Mask" "F.Paste") (roundrect_rratio 0.25) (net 1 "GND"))
  (pad "2" smd roundrect (at 0.9375 0 90) (size 0.975 1.4) (layers "F.Cu" "F.Mask" "F.Paste") (roundrect_rratio 0.25) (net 6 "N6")))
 (gr_rect (start 99.5 58.5) (end 171 71.5) (stroke (width 0.05) (type default)) (fill no) (layer "Edge.Cuts"))
 (segment (start 129.9 66.95) (end 133.3625 66.95) (width 0.2) (layer "F.Cu") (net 4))
 (segment (start 120.5 62.175) (end 105.665 62.175) (width 0.5) (layer "F.Cu") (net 4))
 (segment (start 127.5 64.55) (end 129.9 66.95) (width 0.2) (layer "F.Cu") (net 4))
 (segment (start 132.8625 64.55) (end 133.3625 65.05) (width 0.5) (layer "F.Cu") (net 4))
 (segment (start 120.5 62.175) (end 125.125 62.175) (width 0.5) (layer "F.Cu") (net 4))
 (segment (start 127.5 64.55) (end 132.8625 64.55) (width 0.5) (layer "F.Cu") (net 4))
 (segment (start 105.665 62.175) (end 104.115 63.725) (width 0.5) (layer "F.Cu") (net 4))
 (segment (start 125.125 62.175) (end 127.5 64.55) (width 0.5) (layer "F.Cu") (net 4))
 (segment (start 143.55 63.95) (end 146.4375 61.0625) (width 0.5) (layer "F.Cu") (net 3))
 (segment (start 142.4 65.05) (end 143.5 63.95) (width 0.5) (layer "F.Cu") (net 3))
 (segment (start 165.225 63.725) (end 166.115 63.725) (width 0.2) (layer "F.Cu") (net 3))
 (segment (start 162.5625 61.0625) (end 165.225 63.725) (width 0.5) (layer "F.Cu") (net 3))
 (segment (start 143.5 63.95) (end 143.55 63.95) (width 0.2) (layer "F.Cu") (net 3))
 (segment (start 154.5 61.0625) (end 162.5625 61.0625) (width 0.5) (layer "F.Cu") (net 3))
 (segment (start 146.4375 61.0625) (end 154.5 61.0625) (width 0.5) (layer "F.Cu") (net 3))
 (segment (start 135.6375 65.05) (end 142.4 65.05) (width 0.5) (layer "F.Cu") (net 3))
 (segment (start 135.6375 66.95) (end 143.1 66.95) (width 0.2) (layer "F.Cu") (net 5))
 (segment (start 143.1 66.95) (end 143.5 66.55) (width 0.2) (layer "F.Cu") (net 5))
 (segment (start 120.5 66.65) (end 120.5 64) (width 0.2) (layer "F.Cu") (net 2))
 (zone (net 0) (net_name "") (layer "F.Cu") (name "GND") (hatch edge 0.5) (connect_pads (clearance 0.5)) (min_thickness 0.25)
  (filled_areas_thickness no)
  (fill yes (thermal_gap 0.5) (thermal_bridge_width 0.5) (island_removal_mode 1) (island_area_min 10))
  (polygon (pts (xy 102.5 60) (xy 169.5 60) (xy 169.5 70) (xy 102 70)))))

